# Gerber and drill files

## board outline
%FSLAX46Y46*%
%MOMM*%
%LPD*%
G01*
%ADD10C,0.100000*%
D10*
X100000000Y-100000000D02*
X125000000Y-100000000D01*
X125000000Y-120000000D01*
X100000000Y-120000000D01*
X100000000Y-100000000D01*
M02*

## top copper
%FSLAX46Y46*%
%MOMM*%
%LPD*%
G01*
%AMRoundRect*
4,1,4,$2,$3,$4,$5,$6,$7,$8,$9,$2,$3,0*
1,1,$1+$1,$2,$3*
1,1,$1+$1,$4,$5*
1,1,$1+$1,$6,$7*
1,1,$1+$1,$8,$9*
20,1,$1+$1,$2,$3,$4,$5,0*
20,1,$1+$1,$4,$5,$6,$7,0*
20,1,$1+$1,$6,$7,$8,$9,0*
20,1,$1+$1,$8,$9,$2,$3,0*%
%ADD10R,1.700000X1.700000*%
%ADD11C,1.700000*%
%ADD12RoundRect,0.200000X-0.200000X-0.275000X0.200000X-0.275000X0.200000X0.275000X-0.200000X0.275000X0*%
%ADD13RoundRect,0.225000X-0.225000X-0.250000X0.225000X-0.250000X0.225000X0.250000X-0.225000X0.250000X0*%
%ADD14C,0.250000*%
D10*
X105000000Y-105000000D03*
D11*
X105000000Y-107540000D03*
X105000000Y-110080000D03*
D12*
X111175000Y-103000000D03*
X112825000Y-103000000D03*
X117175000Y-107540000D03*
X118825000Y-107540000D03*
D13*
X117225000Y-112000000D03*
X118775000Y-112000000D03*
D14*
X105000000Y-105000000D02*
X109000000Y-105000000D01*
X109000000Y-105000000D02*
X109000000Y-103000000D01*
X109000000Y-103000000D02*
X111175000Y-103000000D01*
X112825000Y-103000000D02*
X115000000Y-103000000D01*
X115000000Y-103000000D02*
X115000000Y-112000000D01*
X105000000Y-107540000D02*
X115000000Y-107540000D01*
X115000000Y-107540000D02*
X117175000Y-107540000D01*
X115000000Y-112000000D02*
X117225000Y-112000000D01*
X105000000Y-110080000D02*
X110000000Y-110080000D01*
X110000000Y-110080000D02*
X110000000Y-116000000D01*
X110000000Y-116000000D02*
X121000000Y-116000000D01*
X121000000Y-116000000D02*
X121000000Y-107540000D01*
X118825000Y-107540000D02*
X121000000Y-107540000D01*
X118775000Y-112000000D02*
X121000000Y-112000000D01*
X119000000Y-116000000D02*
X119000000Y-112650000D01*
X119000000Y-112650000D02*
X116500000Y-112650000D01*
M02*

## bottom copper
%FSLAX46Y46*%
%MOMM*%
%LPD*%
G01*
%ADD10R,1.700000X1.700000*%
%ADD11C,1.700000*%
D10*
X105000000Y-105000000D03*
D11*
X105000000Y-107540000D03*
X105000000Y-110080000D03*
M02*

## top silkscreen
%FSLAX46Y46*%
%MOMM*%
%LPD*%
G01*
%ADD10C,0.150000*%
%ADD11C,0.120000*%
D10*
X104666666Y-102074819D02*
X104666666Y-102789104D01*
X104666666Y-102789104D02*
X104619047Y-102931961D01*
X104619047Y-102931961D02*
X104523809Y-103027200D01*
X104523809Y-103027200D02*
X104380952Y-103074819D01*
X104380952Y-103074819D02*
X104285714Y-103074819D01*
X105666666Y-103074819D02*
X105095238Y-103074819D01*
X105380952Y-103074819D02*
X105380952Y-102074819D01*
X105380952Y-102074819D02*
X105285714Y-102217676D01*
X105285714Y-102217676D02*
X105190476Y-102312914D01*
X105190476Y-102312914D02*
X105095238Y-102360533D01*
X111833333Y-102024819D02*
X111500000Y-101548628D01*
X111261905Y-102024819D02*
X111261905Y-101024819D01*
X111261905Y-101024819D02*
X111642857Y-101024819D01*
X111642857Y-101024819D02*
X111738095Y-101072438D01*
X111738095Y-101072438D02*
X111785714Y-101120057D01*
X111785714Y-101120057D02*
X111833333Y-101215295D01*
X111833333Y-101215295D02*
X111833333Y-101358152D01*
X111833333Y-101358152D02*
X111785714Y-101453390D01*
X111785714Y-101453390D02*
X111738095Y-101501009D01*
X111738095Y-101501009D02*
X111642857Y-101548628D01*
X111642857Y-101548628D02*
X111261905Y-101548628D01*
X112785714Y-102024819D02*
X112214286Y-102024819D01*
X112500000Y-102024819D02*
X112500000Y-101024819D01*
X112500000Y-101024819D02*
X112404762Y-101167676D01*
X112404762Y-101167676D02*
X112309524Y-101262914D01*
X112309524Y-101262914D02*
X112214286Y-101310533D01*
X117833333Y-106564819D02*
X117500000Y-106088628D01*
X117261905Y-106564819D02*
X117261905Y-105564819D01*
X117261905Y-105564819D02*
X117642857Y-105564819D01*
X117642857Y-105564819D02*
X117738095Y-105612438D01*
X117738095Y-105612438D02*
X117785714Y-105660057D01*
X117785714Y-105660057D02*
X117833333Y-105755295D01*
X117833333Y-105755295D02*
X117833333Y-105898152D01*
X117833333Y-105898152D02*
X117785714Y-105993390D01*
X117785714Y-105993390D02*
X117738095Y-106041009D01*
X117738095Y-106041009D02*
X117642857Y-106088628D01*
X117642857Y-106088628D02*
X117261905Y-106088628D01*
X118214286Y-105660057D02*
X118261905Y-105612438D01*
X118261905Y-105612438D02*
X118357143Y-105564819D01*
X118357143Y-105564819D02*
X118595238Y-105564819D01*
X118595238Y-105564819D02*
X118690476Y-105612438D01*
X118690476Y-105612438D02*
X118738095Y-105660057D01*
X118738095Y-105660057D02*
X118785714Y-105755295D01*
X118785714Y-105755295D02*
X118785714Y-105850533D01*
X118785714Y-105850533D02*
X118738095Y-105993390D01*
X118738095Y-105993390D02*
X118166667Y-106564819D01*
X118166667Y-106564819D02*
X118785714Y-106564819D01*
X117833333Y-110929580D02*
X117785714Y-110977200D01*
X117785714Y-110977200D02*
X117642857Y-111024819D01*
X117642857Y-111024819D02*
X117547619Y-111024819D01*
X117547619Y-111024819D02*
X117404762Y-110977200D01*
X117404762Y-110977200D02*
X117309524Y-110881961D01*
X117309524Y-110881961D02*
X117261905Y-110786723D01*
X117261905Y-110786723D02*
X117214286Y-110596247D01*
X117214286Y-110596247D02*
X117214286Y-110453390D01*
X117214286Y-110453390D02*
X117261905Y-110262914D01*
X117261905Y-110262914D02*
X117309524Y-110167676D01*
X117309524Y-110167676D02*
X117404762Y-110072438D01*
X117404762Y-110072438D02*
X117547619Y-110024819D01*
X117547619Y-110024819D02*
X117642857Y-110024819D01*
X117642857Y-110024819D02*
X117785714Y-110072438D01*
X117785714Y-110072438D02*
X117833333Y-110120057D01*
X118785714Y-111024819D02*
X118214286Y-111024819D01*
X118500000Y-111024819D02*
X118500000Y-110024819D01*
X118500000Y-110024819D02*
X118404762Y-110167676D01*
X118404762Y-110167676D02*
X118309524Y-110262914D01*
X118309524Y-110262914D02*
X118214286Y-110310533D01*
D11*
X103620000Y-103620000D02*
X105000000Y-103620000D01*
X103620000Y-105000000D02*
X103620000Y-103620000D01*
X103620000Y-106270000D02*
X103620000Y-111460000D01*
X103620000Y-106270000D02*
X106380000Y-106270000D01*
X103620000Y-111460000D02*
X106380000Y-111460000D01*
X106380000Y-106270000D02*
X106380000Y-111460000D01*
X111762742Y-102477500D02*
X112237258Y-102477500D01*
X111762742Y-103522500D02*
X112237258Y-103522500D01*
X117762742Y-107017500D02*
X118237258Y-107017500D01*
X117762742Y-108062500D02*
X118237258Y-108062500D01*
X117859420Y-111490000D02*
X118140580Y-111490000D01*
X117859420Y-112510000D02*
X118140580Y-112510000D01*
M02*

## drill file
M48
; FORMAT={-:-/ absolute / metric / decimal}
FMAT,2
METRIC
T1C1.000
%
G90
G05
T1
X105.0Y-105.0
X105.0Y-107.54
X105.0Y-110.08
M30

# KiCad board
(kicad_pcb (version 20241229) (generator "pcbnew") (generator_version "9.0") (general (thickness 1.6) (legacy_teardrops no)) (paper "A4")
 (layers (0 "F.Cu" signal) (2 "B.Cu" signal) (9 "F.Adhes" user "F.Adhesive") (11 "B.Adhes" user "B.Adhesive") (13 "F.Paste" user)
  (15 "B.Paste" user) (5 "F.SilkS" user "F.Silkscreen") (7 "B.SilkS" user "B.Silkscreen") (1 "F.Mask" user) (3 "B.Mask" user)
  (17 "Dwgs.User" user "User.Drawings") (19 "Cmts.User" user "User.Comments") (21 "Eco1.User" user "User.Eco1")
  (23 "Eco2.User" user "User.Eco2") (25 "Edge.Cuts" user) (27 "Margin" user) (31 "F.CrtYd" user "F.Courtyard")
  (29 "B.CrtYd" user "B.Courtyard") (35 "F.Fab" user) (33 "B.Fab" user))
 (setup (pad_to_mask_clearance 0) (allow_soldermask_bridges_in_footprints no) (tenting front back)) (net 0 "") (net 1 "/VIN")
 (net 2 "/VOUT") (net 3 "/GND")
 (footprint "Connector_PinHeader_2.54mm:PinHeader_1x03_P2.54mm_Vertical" (layer "F.Cu") (at 105 105)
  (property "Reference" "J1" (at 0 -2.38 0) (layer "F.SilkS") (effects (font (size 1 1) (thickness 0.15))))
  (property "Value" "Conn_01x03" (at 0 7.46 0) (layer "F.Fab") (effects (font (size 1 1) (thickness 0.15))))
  (fp_line (start -1.38 -1.38) (end 0 -1.38) (stroke (width 0.12) (type solid)) (layer "F.SilkS"))
  (fp_line (start -1.38 0) (end -1.38 -1.38) (stroke (width 0.12) (type solid)) (layer "F.SilkS"))
  (fp_line (start -1.38 1.27) (end -1.38 6.46) (stroke (width 0.12) (type solid)) (layer "F.SilkS"))
  (fp_line (start -1.38 1.27) (end 1.38 1.27) (stroke (width 0.12) (type solid)) (layer "F.SilkS"))
  (fp_line (start -1.38 6.46) (end 1.38 6.46) (stroke (width 0.12) (type solid)) (layer "F.SilkS"))
  (fp_line (start 1.38 1.27) (end 1.38 6.46) (stroke (width 0.12) (type solid)) (layer "F.SilkS"))
  (pad "1" thru_hole rect (at 0 0) (size 1.7 1.7) (drill 1) (layers "*.Cu" "*.Mask") (remove_unused_layers no) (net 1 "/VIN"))
  (pad "2" thru_hole circle (at 0 2.54) (size 1.7 1.7) (drill 1) (layers "*.Cu" "*.Mask") (remove_unused_layers no) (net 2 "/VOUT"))
  (pad "3" thru_hole circle (at 0 5.08) (size 1.7 1.7) (drill 1) (layers "*.Cu" "*.Mask") (remove_unused_layers no) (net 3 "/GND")))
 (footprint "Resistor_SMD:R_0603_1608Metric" (layer "F.Cu") (at 112 103)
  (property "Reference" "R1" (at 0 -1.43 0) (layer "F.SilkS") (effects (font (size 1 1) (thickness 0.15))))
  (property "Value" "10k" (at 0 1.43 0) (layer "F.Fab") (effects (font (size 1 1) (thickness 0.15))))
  (fp_line (start -0.237258 -0.5225) (end 0.237258 -0.5225) (stroke (width 0.12) (type solid)) (layer "F.SilkS"))
  (fp_line (start -0.237258 0.5225) (end 0.237258 0.5225) (stroke (width 0.12) (type solid)) (layer "F.SilkS"))
  (pad "1" smd roundrect (at -0.825 0) (size 0.8 0.95) (layers "F.Cu" "F.Mask" "F.Paste") (roundrect_rratio 0.25) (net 1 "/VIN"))
  (pad "2" smd roundrect (at 0.825 0) (size 0.8 0.95) (layers "F.Cu" "F.Mask" "F.Paste") (roundrect_rratio 0.25) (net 2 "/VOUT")))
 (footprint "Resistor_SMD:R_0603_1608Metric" (layer "F.Cu") (at 118 107.54)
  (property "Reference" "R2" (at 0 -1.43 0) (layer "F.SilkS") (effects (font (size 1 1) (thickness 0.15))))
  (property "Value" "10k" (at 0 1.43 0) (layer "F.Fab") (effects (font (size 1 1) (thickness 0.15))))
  (fp_line (start -0.237258 -0.5225) (end 0.237258 -0.5225) (stroke (width 0.12) (type solid)) (layer "F.SilkS"))
  (fp_line (start -0.237258 0.5225) (end 0.237258 0.5225) (stroke (width 0.12) (type solid)) (layer "F.SilkS"))
  (pad "1" smd roundrect (at -0.825 0) (size 0.8 0.95) (layers "F.Cu" "F.Mask" "F.Paste") (roundrect_rratio 0.25) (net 2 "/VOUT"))
  (pad "2" smd roundrect (at 0.825 0) (size 0.8 0.95) (layers "F.Cu" "F.Mask" "F.Paste") (roundrect_rratio 0.25) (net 3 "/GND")))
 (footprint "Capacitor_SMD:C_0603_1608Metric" (layer "F.Cu") (at 118 112)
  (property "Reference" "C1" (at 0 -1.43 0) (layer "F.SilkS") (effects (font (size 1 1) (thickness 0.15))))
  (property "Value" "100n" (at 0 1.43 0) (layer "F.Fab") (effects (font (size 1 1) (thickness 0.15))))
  (fp_line (start -0.14058 -0.51) (end 0.14058 -0.51) (stroke (width 0.12) (type solid)) (layer "F.SilkS"))
  (fp_line (start -0.14058 0.51) (end 0.14058 0.51) (stroke (width 0.12) (type solid)) (layer "F.SilkS"))
  (pad "1" smd roundrect (at -0.775 0) (size 0.9 0.95) (layers "F.Cu" "F.Mask" "F.Paste") (roundrect_rratio 0.25) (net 2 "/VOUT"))
  (pad "2" smd roundrect (at 0.775 0) (size 0.9 0.95) (layers "F.Cu" "F.Mask" "F.Paste") (roundrect_rratio 0.25) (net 3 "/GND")))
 (gr_rect (start 100 100) (end 125 120) (stroke (width 0.1) (type default)) (fill no) (layer "Edge.Cuts"))
 (segment (start 105 105) (end 109 105) (width 0.25) (layer "F.Cu") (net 1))
 (segment (start 109 105) (end 109 103) (width 0.25) (layer "F.Cu") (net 1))
 (segment (start 109 103) (end 111.175 103) (width 0.25) (layer "F.Cu") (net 1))
 (segment (start 112.825 103) (end 115 103) (width 0.25) (layer "F.Cu") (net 2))
 (segment (start 115 103) (end 115 112) (width 0.25) (layer "F.Cu") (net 2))
 (segment (start 105 107.54) (end 115 107.54) (width 0.25) (layer "F.Cu") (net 2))
 (segment (start 115 107.54) (end 117.175 107.54) (width 0.25) (layer "F.Cu") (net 2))
 (segment (start 115 112) (end 117.225 112) (width 0.25) (layer "F.Cu") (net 2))
 (segment (start 105 110.08) (end 110 110.08) (width 0.25) (layer "F.Cu") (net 3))
 (segment (start 110 110.08) (end 110 116) (width 0.25) (layer "F.Cu") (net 3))
 (segment (start 110 116) (end 121 116) (width 0.25) (layer "F.Cu") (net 3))
 (segment (start 121 116) (end 121 107.54) (width 0.25) (layer "F.Cu") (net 3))
 (segment (start 118.825 107.54) (end 121 107.54) (width 0.25) (layer "F.Cu") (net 3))
 (segment (start 118.775 112) (end 121 112) (width 0.25) (layer "F.Cu") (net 3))
 (segment (start 119 116) (end 119 112.65) (width 0.25) (layer "F.Cu") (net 3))
 (segment (start 119 112.65) (end 116.5 112.65) (width 0.25) (layer "F.Cu") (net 3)))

